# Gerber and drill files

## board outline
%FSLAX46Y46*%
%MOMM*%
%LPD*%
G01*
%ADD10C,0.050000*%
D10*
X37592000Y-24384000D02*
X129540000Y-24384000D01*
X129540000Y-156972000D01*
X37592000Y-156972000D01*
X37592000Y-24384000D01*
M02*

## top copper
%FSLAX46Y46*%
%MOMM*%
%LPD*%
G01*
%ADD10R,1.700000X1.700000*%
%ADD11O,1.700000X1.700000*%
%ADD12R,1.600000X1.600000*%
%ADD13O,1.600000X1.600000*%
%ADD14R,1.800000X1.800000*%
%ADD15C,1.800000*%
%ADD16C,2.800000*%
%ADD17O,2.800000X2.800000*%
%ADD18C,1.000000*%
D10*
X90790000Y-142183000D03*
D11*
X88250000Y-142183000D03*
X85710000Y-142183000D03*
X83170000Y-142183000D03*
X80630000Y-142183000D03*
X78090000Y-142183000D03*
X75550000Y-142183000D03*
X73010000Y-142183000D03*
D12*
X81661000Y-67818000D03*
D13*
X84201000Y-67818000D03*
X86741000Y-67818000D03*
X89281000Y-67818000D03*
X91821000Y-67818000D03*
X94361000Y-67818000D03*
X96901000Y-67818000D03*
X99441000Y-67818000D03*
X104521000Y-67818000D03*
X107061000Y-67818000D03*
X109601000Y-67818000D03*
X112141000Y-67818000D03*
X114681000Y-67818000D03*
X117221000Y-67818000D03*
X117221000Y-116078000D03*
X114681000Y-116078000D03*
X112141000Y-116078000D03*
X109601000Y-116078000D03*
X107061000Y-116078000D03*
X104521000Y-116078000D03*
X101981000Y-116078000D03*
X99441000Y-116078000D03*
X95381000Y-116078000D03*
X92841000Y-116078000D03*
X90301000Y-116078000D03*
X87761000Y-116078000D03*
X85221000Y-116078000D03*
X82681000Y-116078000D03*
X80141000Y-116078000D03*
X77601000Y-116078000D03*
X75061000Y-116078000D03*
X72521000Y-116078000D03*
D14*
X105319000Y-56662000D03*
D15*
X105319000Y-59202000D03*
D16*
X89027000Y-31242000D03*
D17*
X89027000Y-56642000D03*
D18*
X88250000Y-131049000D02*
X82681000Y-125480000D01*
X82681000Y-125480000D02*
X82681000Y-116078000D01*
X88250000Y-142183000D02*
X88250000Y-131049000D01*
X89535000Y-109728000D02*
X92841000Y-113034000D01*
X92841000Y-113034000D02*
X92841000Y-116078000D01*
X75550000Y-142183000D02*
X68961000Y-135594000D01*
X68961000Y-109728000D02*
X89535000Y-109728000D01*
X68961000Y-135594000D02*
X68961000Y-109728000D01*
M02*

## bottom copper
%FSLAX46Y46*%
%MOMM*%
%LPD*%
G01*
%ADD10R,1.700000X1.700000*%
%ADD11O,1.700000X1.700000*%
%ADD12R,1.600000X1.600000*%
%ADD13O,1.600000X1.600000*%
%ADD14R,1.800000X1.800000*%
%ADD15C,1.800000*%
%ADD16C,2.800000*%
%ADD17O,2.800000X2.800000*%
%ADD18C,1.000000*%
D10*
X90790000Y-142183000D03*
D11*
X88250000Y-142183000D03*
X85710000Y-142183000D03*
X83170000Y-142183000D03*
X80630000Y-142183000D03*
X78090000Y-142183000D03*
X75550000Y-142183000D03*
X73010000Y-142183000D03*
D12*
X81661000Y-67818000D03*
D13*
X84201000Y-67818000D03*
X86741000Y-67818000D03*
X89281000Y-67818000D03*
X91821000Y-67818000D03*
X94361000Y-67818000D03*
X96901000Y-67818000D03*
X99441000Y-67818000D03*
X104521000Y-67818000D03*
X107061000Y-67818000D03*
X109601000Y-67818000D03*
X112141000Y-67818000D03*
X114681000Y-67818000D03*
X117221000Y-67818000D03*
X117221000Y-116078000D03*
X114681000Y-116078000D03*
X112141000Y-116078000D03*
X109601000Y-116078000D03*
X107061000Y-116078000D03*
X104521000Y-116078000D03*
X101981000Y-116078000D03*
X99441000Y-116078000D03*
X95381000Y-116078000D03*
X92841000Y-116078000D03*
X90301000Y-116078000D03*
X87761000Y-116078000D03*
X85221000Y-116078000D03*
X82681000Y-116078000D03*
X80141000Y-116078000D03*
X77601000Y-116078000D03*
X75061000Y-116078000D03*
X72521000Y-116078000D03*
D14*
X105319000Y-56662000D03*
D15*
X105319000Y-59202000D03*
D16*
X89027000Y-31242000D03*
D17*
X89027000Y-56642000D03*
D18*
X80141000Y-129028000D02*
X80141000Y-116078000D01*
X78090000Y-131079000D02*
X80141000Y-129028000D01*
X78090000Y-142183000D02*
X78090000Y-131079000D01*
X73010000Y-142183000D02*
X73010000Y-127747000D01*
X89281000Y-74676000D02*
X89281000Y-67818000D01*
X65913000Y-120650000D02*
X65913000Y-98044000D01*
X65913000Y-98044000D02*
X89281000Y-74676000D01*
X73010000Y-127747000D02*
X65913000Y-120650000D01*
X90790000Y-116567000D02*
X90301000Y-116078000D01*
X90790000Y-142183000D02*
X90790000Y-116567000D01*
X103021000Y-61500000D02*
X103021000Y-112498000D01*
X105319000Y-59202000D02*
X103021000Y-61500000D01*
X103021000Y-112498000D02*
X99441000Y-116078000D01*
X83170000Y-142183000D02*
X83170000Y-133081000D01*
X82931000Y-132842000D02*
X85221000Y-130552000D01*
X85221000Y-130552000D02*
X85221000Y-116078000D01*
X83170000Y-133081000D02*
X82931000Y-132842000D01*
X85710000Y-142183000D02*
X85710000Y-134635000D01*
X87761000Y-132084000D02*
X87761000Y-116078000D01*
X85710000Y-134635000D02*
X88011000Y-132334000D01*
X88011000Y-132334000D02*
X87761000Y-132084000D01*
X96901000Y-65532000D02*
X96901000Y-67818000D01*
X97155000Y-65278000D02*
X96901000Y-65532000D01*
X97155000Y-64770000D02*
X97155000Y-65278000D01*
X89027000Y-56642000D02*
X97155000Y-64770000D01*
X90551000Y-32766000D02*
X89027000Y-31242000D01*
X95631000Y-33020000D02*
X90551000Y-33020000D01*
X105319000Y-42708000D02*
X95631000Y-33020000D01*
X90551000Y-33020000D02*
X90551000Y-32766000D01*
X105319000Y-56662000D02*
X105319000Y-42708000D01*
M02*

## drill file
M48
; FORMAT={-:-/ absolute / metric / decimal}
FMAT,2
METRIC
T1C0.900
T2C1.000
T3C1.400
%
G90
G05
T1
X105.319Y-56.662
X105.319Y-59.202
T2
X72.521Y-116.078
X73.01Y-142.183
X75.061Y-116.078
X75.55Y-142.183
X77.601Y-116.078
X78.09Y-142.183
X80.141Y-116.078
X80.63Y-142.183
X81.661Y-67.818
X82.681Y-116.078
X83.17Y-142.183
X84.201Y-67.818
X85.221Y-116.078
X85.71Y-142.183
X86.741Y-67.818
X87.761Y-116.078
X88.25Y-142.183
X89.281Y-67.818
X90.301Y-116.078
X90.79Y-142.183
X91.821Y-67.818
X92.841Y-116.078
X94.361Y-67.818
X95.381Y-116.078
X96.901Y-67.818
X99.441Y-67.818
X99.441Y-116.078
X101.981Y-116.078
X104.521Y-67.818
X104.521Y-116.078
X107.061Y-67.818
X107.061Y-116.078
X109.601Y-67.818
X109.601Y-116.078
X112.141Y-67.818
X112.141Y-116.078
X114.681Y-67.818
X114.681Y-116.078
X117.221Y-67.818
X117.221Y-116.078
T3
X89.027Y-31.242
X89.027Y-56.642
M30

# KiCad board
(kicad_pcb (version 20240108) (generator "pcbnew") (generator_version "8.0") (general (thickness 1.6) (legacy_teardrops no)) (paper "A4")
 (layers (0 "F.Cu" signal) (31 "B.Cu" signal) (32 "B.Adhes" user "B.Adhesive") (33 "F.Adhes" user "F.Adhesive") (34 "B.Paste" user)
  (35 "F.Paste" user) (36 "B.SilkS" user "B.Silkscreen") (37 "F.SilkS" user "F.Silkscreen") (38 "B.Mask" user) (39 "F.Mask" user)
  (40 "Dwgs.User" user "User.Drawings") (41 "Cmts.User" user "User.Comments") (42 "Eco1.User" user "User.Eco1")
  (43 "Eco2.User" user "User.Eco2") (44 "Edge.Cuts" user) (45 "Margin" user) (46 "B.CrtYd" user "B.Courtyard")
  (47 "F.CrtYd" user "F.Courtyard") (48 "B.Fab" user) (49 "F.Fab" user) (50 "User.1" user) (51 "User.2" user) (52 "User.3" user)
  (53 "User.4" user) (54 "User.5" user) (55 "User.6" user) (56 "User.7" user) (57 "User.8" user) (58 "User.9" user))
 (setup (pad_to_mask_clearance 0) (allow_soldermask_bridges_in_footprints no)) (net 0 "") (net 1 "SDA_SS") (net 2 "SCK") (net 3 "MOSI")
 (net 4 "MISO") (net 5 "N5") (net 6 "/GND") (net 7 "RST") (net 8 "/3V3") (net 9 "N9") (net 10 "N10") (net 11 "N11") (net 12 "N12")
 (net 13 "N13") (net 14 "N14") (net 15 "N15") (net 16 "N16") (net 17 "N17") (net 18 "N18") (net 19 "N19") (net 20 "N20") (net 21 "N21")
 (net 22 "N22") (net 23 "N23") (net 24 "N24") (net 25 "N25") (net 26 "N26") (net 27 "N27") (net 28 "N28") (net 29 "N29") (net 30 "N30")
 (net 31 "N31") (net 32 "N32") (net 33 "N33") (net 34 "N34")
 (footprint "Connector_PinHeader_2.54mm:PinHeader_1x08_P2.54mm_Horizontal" (layer "F.Cu") (at 90.79 142.183 -90)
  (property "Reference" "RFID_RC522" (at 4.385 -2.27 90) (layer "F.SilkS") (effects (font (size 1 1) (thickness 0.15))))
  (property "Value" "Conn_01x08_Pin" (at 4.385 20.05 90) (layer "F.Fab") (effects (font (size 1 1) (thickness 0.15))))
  (pad "1" thru_hole rect (at 0 0 270) (size 1.7 1.7) (drill 1) (layers "*.Cu" "*.Mask") (remove_unused_layers no) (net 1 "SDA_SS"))
  (pad "2" thru_hole oval (at 0 2.54 270) (size 1.7 1.7) (drill 1) (layers "*.Cu" "*.Mask") (remove_unused_layers no) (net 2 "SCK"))
  (pad "3" thru_hole oval (at 0 5.08 270) (size 1.7 1.7) (drill 1) (layers "*.Cu" "*.Mask") (remove_unused_layers no) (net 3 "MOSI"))
  (pad "4" thru_hole oval (at 0 7.62 270) (size 1.7 1.7) (drill 1) (layers "*.Cu" "*.Mask") (remove_unused_layers no) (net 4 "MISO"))
  (pad "5" thru_hole oval (at 0 10.16 270) (size 1.7 1.7) (drill 1) (layers "*.Cu" "*.Mask") (remove_unused_layers no) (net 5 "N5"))
  (pad "6" thru_hole oval (at 0 12.7 270) (size 1.7 1.7) (drill 1) (layers "*.Cu" "*.Mask") (remove_unused_layers no) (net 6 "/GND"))
  (pad "7" thru_hole oval (at 0 15.24 270) (size 1.7 1.7) (drill 1) (layers "*.Cu" "*.Mask") (remove_unused_layers no) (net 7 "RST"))
  (pad "8" thru_hole oval (at 0 17.78 270) (size 1.7 1.7) (drill 1) (layers "*.Cu" "*.Mask") (remove_unused_layers no) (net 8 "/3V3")))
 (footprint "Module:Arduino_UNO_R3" (layer "F.Cu") (at 81.661 67.818)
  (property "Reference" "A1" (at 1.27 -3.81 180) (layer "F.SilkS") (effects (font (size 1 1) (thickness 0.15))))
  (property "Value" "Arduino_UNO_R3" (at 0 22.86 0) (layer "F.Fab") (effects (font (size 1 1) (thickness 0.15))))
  (pad "1" thru_hole rect (at 0 0 90) (size 1.6 1.6) (drill 1) (layers "*.Cu" "*.Mask") (remove_unused_layers no) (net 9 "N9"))
  (pad "2" thru_hole oval (at 2.54 0 90) (size 1.6 1.6) (drill 1) (layers "*.Cu" "*.Mask") (remove_unused_layers no) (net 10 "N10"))
  (pad "3" thru_hole oval (at 5.08 0 90) (size 1.6 1.6) (drill 1) (layers "*.Cu" "*.Mask") (remove_unused_layers no) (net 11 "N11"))
  (pad "4" thru_hole oval (at 7.62 0 90) (size 1.6 1.6) (drill 1) (layers "*.Cu" "*.Mask") (remove_unused_layers no) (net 8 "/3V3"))
  (pad "5" thru_hole oval (at 10.16 0 90) (size 1.6 1.6) (drill 1) (layers "*.Cu" "*.Mask") (remove_unused_layers no) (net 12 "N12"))
  (pad "6" thru_hole oval (at 12.7 0 90) (size 1.6 1.6) (drill 1) (layers "*.Cu" "*.Mask") (remove_unused_layers no) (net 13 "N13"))
  (pad "7" thru_hole oval (at 15.24 0 90) (size 1.6 1.6) (drill 1) (layers "*.Cu" "*.Mask") (remove_unused_layers no) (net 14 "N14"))
  (pad "8" thru_hole oval (at 17.78 0 90) (size 1.6 1.6) (drill 1) (layers "*.Cu" "*.Mask") (remove_unused_layers no) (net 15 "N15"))
  (pad "9" thru_hole oval (at 22.86 0 90) (size 1.6 1.6) (drill 1) (layers "*.Cu" "*.Mask") (remove_unused_layers no) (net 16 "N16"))
  (pad "10" thru_hole oval (at 25.4 0 90) (size 1.6 1.6) (drill 1) (layers "*.Cu" "*.Mask") (remove_unused_layers no) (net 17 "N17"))
  (pad "11" thru_hole oval (at 27.94 0 90) (size 1.6 1.6) (drill 1) (layers "*.Cu" "*.Mask") (remove_unused_layers no) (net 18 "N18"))
  (pad "12" thru_hole oval (at 30.48 0 90) (size 1.6 1.6) (drill 1) (layers "*.Cu" "*.Mask") (remove_unused_layers no) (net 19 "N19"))
  (pad "13" thru_hole oval (at 33.02 0 90) (size 1.6 1.6) (drill 1) (layers "*.Cu" "*.Mask") (remove_unused_layers no) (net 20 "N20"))
  (pad "14" thru_hole oval (at 35.56 0 90) (size 1.6 1.6) (drill 1) (layers "*.Cu" "*.Mask") (remove_unused_layers no) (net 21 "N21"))
  (pad "15" thru_hole oval (at 35.56 48.26 90) (size 1.6 1.6) (drill 1) (layers "*.Cu" "*.Mask") (remove_unused_layers no) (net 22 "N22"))
  (pad "16" thru_hole oval (at 33.02 48.26 90) (size 1.6 1.6) (drill 1) (layers "*.Cu" "*.Mask") (remove_unused_layers no) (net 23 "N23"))
  (pad "17" thru_hole oval (at 30.48 48.26 90) (size 1.6 1.6) (drill 1) (layers "*.Cu" "*.Mask") (remove_unused_layers no) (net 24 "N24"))
  (pad "18" thru_hole oval (at 27.94 48.26 90) (size 1.6 1.6) (drill 1) (layers "*.Cu" "*.Mask") (remove_unused_layers no) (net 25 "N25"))
  (pad "19" thru_hole oval (at 25.4 48.26 90) (size 1.6 1.6) (drill 1) (layers "*.Cu" "*.Mask") (remove_unused_layers no) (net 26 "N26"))
  (pad "20" thru_hole oval (at 22.86 48.26 90) (size 1.6 1.6) (drill 1) (layers "*.Cu" "*.Mask") (remove_unused_layers no) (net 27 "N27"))
  (pad "21" thru_hole oval (at 20.32 48.26 90) (size 1.6 1.6) (drill 1) (layers "*.Cu" "*.Mask") (remove_unused_layers no) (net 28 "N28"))
  (pad "22" thru_hole oval (at 17.78 48.26 90) (size 1.6 1.6) (drill 1) (layers "*.Cu" "*.Mask") (remove_unused_layers no) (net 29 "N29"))
  (pad "23" thru_hole oval (at 13.72 48.26 90) (size 1.6 1.6) (drill 1) (layers "*.Cu" "*.Mask") (remove_unused_layers no) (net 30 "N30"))
  (pad "24" thru_hole oval (at 11.18 48.26 90) (size 1.6 1.6) (drill 1) (layers "*.Cu" "*.Mask") (remove_unused_layers no) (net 7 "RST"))
  (pad "25" thru_hole oval (at 8.64 48.26 90) (size 1.6 1.6) (drill 1) (layers "*.Cu" "*.Mask") (remove_unused_layers no) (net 1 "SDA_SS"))
  (pad "26" thru_hole oval (at 6.1 48.26 90) (size 1.6 1.6) (drill 1) (layers "*.Cu" "*.Mask") (remove_unused_layers no) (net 3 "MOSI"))
  (pad "27" thru_hole oval (at 3.56 48.26 90) (size 1.6 1.6) (drill 1) (layers "*.Cu" "*.Mask") (remove_unused_layers no) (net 4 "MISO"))
  (pad "28" thru_hole oval (at 1.02 48.26 90) (size 1.6 1.6) (drill 1) (layers "*.Cu" "*.Mask") (remove_unused_layers no) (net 2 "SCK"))
  (pad "29" thru_hole oval (at -1.52 48.26 90) (size 1.6 1.6) (drill 1) (layers "*.Cu" "*.Mask") (remove_unused_layers no) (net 6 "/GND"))
  (pad "30" thru_hole oval (at -4.06 48.26 90) (size 1.6 1.6) (drill 1) (layers "*.Cu" "*.Mask") (remove_unused_layers no) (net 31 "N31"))
  (pad "31" thru_hole oval (at -6.6 48.26 90) (size 1.6 1.6) (drill 1) (layers "*.Cu" "*.Mask") (remove_unused_layers no) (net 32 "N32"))
  (pad "32" thru_hole oval (at -9.14 48.26 90) (size 1.6 1.6) (drill 1) (layers "*.Cu" "*.Mask") (remove_unused_layers no) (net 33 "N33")))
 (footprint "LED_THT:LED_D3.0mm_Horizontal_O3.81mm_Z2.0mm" (layer "F.Cu") (at 105.319 56.662 -90)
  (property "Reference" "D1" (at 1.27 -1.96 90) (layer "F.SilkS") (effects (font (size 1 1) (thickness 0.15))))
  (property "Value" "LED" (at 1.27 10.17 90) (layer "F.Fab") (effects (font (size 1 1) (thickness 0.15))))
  (pad "1" thru_hole rect (at 0 0 270) (size 1.8 1.8) (drill 0.9) (layers "*.Cu" "*.Mask") (remove_unused_layers no) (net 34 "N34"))
  (pad "2" thru_hole circle (at 2.54 0 270) (size 1.8 1.8) (drill 0.9) (layers "*.Cu" "*.Mask") (remove_unused_layers no) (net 29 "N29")))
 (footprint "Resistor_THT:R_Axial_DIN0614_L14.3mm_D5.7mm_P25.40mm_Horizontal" (layer "F.Cu") (at 89.027 31.242 -90)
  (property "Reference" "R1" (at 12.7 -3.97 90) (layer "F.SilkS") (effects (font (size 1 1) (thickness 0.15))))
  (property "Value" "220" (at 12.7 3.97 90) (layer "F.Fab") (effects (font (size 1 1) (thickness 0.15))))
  (pad "1" thru_hole circle (at 0 0 270) (size 2.8 2.8) (drill 1.4) (layers "*.Cu" "*.Mask") (remove_unused_layers no) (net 34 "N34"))
  (pad "2" thru_hole oval (at 25.4 0 270) (size 2.8 2.8) (drill 1.4) (layers "*.Cu" "*.Mask") (remove_unused_layers no) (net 14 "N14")))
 (gr_rect (start 37.592 24.384) (end 129.54 156.972) (stroke (width 0.05) (type default)) (fill none) (layer "Edge.Cuts"))
 (segment (start 80.141 129.028) (end 80.141 116.078) (width 1) (layer "B.Cu") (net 6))
 (segment (start 78.09 131.079) (end 80.141 129.028) (width 1) (layer "B.Cu") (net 6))
 (segment (start 78.09 142.183) (end 78.09 131.079) (width 1) (layer "B.Cu") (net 6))
 (segment (start 73.01 142.183) (end 73.01 127.747) (width 1) (layer "B.Cu") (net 8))
 (segment (start 89.281 74.676) (end 89.281 67.818) (width 1) (layer "B.Cu") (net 8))
 (segment (start 65.913 120.65) (end 65.913 98.044) (width 1) (layer "B.Cu") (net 8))
 (segment (start 65.913 98.044) (end 89.281 74.676) (width 1) (layer "B.Cu") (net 8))
 (segment (start 73.01 127.747) (end 65.913 120.65) (width 1) (layer "B.Cu") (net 8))
 (segment (start 90.79 116.567) (end 90.301 116.078) (width 1) (layer "B.Cu") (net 1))
 (segment (start 90.79 142.183) (end 90.79 116.567) (width 1) (layer "B.Cu") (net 1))
 (segment (start 103.021 61.5) (end 103.021 112.498) (width 1) (layer "B.Cu") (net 29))
 (segment (start 105.319 59.202) (end 103.021 61.5) (width 1) (layer "B.Cu") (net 29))
 (segment (start 103.021 112.498) (end 99.441 116.078) (width 1) (layer "B.Cu") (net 29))
 (segment (start 83.17 142.183) (end 83.17 133.081) (width 1) (layer "B.Cu") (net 4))
 (segment (start 82.931 132.842) (end 85.221 130.552) (width 1) (layer "B.Cu") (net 4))
 (segment (start 85.221 130.552) (end 85.221 116.078) (width 1) (layer "B.Cu") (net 4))
 (segment (start 83.17 133.081) (end 82.931 132.842) (width 1) (layer "B.Cu") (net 4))
 (segment (start 85.71 142.183) (end 85.71 134.635) (width 1) (layer "B.Cu") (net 3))
 (segment (start 87.761 132.084) (end 87.761 116.078) (width 1) (layer "B.Cu") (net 3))
 (segment (start 85.71 134.635) (end 88.011 132.334) (width 1) (layer "B.Cu") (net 3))
 (segment (start 88.011 132.334) (end 87.761 132.084) (width 1) (layer "B.Cu") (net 3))
 (segment (start 88.25 131.049) (end 82.681 125.48) (width 1) (layer "F.Cu") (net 2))
 (segment (start 82.681 125.48) (end 82.681 116.078) (width 1) (layer "F.Cu") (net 2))
 (segment (start 88.25 142.183) (end 88.25 131.049) (width 1) (layer "F.Cu") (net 2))
 (segment (start 96.901 65.532) (end 96.901 67.818) (width 1) (layer "B.Cu") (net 14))
 (segment (start 97.155 65.278) (end 96.901 65.532) (width 1) (layer "B.Cu") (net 14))
 (segment (start 97.155 64.77) (end 97.155 65.278) (width 1) (layer "B.Cu") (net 14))
 (segment (start 89.027 56.642) (end 97.155 64.77) (width 1) (layer "B.Cu") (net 14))
 (segment (start 89.535 109.728) (end 92.841 113.034) (width 1) (layer "F.Cu") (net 7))
 (segment (start 92.841 113.034) (end 92.841 116.078) (width 1) (layer "F.Cu") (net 7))
 (segment (start 75.55 142.183) (end 68.961 135.594) (width 1) (layer "F.Cu") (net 7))
 (segment (start 68.961 109.728) (end 89.535 109.728) (width 1) (layer "F.Cu") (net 7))
 (segment (start 68.961 135.594) (end 68.961 109.728) (width 1) (layer "F.Cu") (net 7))
 (segment (start 90.551 32.766) (end 89.027 31.242) (width 1) (layer "B.Cu") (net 34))
 (segment (start 95.631 33.02) (end 90.551 33.02) (width 1) (layer "B.Cu") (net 34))
 (segment (start 105.319 42.708) (end 95.631 33.02) (width 1) (layer "B.Cu") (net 34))
 (segment (start 90.551 33.02) (end 90.551 32.766) (width 1) (layer "B.Cu") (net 34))
 (segment (start 105.319 56.662) (end 105.319 42.708) (width 1) (layer "B.Cu") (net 34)))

